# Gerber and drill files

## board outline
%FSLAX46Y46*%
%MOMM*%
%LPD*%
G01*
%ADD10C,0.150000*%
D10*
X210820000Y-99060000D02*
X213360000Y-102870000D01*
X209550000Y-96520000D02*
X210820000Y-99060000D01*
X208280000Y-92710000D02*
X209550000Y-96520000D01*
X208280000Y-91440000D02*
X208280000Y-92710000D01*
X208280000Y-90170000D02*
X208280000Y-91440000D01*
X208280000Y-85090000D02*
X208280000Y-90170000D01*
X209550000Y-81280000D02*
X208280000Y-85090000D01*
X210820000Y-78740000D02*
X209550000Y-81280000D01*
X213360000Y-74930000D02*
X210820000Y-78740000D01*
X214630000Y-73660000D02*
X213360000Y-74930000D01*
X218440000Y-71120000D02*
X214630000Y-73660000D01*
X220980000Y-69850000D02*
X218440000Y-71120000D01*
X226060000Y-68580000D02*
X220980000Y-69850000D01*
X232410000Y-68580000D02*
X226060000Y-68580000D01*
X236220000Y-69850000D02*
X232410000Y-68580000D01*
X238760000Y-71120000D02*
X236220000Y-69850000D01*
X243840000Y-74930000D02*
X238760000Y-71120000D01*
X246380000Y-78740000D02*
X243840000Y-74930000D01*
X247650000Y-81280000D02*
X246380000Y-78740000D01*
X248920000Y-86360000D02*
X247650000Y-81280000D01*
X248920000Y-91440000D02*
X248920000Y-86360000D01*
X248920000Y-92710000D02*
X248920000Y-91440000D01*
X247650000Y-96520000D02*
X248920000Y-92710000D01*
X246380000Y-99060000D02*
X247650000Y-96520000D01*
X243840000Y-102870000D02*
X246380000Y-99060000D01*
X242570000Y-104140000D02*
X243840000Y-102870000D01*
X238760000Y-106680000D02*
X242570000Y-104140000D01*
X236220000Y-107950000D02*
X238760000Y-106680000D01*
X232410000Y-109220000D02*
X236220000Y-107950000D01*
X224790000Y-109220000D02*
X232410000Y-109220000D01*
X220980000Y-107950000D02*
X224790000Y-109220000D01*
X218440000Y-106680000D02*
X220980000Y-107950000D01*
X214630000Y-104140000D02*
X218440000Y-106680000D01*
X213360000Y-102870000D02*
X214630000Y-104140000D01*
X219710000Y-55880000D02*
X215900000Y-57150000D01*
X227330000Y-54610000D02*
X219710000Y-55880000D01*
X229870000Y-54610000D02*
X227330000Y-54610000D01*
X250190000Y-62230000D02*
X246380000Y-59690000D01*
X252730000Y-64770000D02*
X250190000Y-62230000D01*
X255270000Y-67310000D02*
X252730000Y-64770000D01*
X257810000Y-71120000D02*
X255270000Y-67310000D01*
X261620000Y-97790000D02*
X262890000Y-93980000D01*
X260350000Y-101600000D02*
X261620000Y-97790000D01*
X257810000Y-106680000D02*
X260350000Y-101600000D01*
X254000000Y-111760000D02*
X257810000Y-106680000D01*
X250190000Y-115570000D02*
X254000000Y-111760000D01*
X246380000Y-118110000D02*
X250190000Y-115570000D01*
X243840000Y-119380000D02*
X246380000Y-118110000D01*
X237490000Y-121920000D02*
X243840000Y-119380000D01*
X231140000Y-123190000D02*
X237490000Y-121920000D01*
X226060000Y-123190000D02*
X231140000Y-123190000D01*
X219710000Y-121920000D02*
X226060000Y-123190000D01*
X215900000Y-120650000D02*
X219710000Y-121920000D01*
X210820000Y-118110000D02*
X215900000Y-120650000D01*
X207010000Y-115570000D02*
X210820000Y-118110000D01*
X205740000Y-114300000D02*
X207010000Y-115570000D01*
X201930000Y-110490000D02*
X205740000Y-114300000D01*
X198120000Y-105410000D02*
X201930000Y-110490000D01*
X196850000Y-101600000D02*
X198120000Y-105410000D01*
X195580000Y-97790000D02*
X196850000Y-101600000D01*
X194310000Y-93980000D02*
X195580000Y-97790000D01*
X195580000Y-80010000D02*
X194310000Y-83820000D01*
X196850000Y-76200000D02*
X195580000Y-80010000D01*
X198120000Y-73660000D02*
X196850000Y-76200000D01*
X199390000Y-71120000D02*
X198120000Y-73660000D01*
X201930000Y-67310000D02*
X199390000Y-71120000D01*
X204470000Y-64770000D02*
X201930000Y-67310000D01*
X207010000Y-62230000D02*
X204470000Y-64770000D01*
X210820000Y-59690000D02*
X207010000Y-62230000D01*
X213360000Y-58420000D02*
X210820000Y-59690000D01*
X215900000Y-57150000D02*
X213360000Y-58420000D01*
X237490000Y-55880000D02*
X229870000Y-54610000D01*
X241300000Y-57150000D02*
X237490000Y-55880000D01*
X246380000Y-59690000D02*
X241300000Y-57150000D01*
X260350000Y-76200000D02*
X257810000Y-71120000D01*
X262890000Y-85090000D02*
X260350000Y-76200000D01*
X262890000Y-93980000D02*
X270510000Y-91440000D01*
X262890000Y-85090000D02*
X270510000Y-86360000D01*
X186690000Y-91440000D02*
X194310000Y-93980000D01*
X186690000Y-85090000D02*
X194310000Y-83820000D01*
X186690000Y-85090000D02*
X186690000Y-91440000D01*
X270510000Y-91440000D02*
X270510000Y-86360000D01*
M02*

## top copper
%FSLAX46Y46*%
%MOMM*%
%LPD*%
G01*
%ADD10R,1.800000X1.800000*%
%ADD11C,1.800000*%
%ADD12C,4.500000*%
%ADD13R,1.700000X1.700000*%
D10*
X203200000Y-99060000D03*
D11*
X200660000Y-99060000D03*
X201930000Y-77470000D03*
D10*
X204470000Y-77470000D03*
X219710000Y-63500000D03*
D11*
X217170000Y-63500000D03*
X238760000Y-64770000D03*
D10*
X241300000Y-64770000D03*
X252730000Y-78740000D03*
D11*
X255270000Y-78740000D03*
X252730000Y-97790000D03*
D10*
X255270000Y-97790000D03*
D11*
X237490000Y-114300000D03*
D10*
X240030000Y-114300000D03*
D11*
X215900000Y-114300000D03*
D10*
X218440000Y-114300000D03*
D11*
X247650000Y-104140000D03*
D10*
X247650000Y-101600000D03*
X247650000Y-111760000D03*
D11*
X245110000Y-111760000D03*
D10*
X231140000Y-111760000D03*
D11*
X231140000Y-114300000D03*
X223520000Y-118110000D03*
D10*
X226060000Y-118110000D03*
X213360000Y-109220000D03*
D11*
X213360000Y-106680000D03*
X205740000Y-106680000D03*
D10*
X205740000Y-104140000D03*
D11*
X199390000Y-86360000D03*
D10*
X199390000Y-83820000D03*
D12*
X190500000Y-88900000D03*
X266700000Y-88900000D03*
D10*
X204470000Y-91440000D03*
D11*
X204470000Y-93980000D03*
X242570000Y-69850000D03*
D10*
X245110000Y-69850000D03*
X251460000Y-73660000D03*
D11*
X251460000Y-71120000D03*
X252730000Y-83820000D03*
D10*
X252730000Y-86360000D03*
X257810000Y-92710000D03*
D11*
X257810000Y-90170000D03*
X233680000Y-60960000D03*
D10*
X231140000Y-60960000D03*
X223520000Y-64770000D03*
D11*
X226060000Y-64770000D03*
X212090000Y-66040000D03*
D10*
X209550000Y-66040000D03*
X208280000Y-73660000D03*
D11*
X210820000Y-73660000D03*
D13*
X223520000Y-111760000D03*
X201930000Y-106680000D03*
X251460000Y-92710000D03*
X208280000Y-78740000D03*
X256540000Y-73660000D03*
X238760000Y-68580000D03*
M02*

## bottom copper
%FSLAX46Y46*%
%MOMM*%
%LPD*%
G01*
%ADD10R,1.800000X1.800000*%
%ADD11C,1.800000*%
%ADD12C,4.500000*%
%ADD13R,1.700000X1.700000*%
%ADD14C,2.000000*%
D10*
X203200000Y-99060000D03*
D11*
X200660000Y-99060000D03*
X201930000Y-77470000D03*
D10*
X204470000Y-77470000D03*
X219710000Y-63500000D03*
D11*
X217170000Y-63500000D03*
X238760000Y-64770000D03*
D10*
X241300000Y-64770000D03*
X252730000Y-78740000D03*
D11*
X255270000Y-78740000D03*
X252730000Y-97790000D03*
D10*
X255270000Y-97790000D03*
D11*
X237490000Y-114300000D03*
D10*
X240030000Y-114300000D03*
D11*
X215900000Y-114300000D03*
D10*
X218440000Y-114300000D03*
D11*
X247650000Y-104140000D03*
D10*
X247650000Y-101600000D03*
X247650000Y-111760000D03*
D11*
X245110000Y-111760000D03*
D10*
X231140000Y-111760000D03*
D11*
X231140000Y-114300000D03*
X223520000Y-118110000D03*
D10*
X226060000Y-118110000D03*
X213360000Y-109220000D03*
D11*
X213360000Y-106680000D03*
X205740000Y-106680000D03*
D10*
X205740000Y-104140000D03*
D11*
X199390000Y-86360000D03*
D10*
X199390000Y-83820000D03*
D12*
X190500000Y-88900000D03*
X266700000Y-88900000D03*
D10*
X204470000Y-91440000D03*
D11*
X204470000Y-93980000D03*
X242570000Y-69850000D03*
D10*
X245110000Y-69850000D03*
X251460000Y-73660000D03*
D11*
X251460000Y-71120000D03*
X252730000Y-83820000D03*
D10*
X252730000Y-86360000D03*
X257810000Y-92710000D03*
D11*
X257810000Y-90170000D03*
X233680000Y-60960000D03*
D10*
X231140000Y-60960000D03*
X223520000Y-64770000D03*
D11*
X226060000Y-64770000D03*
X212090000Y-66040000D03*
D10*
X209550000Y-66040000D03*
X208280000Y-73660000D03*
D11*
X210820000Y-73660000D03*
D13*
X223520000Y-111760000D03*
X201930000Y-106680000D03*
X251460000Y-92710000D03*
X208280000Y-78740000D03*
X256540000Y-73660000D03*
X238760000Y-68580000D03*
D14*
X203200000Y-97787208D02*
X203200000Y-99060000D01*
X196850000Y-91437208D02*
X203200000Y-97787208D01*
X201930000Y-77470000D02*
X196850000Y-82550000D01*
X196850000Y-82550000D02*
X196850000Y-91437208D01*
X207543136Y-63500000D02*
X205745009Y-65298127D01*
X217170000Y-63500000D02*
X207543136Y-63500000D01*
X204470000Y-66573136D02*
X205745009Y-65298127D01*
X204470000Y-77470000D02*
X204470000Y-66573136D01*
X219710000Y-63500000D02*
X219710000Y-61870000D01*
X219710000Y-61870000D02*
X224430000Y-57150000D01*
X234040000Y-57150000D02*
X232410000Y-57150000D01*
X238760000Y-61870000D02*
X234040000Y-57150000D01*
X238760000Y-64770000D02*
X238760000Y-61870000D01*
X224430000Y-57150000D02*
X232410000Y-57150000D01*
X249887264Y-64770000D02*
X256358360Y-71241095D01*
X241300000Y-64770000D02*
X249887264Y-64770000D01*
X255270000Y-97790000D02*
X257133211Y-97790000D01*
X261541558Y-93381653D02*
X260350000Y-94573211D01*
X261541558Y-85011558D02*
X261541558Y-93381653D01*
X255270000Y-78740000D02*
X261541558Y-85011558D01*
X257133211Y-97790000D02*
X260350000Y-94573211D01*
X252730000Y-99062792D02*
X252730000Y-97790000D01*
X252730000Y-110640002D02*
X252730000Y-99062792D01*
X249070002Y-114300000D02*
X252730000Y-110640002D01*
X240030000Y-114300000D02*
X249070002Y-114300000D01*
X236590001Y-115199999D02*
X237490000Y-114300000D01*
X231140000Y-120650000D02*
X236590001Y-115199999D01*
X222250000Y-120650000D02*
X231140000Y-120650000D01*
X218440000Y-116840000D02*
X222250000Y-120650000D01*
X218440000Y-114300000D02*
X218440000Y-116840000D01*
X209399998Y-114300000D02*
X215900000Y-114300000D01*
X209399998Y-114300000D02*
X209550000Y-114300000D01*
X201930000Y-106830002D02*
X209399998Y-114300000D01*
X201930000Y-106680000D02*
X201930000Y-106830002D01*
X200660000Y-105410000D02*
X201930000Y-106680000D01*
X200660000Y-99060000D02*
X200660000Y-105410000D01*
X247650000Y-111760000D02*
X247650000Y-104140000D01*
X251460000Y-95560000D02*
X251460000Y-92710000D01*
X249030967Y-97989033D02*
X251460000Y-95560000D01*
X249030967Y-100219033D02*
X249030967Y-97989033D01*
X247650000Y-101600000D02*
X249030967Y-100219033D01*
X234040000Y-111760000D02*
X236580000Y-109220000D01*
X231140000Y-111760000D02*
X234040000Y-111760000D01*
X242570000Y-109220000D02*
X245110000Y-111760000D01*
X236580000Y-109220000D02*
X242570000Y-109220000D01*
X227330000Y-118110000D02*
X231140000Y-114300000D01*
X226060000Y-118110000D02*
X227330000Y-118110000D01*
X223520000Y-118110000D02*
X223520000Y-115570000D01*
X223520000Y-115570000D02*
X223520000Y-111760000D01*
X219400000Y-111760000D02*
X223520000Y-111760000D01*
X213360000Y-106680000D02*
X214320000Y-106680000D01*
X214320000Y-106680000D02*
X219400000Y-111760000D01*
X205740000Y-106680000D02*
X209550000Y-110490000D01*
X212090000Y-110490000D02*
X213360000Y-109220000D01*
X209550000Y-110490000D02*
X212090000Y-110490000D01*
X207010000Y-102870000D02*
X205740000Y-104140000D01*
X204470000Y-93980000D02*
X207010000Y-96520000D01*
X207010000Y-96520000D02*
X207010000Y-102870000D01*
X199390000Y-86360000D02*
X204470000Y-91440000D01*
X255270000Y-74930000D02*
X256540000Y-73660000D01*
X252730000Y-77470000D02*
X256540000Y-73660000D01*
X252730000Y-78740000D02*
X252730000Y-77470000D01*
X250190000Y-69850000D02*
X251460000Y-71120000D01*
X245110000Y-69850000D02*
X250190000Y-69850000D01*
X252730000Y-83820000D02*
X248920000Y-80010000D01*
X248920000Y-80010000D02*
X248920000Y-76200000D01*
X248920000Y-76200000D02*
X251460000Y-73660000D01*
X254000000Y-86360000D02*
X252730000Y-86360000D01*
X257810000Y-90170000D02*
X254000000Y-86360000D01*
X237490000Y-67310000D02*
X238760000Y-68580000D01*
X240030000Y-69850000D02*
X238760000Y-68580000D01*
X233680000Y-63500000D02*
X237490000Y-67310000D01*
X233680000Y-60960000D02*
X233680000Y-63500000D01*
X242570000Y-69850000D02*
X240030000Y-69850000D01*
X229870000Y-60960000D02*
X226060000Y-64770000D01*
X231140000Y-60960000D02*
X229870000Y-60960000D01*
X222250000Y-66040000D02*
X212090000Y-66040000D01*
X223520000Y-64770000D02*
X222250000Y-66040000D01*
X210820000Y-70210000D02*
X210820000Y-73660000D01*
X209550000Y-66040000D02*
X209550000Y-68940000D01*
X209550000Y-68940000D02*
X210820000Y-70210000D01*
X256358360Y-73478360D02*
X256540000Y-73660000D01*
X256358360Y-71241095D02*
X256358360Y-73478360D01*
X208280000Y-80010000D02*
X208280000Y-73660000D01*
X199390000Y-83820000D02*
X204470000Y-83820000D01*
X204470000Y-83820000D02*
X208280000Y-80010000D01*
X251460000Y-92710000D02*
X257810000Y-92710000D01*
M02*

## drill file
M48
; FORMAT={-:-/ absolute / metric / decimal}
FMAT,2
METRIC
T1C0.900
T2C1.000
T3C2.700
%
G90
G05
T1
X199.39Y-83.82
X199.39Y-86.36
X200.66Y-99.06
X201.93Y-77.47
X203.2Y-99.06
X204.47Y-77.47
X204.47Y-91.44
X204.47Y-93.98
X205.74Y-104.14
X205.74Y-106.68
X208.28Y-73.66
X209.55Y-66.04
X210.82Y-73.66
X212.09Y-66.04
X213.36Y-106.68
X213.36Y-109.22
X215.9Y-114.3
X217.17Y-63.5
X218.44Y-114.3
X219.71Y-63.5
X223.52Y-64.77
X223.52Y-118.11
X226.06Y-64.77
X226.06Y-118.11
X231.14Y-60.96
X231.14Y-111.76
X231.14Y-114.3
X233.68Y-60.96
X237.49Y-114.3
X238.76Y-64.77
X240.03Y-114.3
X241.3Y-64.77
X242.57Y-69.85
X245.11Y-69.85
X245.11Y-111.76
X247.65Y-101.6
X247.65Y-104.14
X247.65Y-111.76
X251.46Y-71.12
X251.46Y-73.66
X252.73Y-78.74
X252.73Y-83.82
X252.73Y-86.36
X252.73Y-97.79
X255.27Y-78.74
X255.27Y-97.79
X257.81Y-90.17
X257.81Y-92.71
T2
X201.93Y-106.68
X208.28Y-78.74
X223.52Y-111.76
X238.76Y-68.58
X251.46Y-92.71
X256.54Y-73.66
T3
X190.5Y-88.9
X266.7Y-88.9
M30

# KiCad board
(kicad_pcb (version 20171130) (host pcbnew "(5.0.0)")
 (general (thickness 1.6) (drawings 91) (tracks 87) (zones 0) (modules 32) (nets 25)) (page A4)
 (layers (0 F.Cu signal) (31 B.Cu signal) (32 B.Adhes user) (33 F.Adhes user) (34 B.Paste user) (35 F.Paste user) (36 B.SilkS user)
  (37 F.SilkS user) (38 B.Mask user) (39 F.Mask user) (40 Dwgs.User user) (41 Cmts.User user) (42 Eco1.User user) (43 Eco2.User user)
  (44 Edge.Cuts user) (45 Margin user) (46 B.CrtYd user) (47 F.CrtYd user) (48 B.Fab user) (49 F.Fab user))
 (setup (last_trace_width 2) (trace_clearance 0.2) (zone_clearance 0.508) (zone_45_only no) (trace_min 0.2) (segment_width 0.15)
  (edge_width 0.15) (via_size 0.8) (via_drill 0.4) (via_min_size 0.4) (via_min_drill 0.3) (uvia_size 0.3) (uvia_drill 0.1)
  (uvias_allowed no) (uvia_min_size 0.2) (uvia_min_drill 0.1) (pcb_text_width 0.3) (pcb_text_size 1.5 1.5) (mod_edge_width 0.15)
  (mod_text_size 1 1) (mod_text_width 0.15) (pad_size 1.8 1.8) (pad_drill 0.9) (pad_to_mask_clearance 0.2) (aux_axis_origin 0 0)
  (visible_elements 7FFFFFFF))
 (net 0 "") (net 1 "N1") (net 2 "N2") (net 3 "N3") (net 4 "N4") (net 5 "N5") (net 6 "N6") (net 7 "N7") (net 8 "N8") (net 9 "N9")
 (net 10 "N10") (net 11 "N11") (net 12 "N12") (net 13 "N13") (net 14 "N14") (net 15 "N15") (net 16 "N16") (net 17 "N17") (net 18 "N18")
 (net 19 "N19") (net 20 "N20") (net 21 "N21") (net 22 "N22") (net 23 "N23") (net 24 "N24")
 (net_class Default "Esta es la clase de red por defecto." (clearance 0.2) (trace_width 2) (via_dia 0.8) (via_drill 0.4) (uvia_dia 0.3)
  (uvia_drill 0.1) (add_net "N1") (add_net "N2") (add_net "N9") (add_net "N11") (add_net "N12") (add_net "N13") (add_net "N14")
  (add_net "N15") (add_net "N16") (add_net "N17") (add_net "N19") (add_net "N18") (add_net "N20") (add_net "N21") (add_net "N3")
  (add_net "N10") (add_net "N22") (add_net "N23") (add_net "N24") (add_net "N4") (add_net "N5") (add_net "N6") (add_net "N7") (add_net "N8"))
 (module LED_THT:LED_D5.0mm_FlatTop (layer F.Cu) (at 203.2 99.06 180)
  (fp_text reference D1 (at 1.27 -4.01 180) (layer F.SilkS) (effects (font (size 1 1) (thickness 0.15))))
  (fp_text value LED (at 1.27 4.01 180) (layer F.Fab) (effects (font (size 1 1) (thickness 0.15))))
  (pad 1 thru_hole rect (at 0 0 180) (size 1.8 1.8) (drill 0.9) (layers *.Cu *.Mask) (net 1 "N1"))
  (pad 2 thru_hole circle (at 2.54 0 180) (size 1.8 1.8) (drill 0.9) (layers *.Cu *.Mask) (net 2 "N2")))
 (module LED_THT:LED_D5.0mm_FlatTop (layer F.Cu) (at 204.47 77.47 180)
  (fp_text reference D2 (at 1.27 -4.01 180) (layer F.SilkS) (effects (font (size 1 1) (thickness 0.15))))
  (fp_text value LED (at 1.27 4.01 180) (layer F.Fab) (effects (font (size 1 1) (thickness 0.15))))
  (pad 2 thru_hole circle (at 2.54 0 180) (size 1.8 1.8) (drill 0.9) (layers *.Cu *.Mask) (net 1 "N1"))
  (pad 1 thru_hole rect (at 0 0 180) (size 1.8 1.8) (drill 0.9) (layers *.Cu *.Mask) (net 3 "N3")))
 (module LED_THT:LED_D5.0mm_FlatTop (layer F.Cu) (at 219.71 63.5 180)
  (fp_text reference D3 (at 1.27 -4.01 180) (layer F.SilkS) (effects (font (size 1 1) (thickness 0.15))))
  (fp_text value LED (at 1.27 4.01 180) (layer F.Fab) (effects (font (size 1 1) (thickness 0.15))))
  (pad 1 thru_hole rect (at 0 0 180) (size 1.8 1.8) (drill 0.9) (layers *.Cu *.Mask) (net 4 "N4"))
  (pad 2 thru_hole circle (at 2.54 0 180) (size 1.8 1.8) (drill 0.9) (layers *.Cu *.Mask) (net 3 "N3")))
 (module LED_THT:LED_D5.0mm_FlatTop (layer F.Cu) (at 241.3 64.77 180)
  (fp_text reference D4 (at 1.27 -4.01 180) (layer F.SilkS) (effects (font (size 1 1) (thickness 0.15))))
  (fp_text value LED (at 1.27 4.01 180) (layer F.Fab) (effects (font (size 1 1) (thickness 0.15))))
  (pad 2 thru_hole circle (at 2.54 0 180) (size 1.8 1.8) (drill 0.9) (layers *.Cu *.Mask) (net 4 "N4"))
  (pad 1 thru_hole rect (at 0 0 180) (size 1.8 1.8) (drill 0.9) (layers *.Cu *.Mask) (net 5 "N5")))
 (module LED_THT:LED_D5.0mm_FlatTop (layer F.Cu) (at 252.73 78.74)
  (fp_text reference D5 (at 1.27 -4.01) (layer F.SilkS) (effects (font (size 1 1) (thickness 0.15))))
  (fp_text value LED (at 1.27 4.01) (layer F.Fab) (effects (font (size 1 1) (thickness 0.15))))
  (pad 1 thru_hole rect (at 0 0) (size 1.8 1.8) (drill 0.9) (layers *.Cu *.Mask) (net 5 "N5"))
  (pad 2 thru_hole circle (at 2.54 0) (size 1.8 1.8) (drill 0.9) (layers *.Cu *.Mask) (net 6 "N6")))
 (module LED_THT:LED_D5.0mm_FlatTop (layer F.Cu) (at 255.27 97.79 180)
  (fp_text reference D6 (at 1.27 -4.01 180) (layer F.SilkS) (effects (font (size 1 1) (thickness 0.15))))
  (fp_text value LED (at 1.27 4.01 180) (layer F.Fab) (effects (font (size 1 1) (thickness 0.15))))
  (pad 2 thru_hole circle (at 2.54 0 180) (size 1.8 1.8) (drill 0.9) (layers *.Cu *.Mask) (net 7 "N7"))
  (pad 1 thru_hole rect (at 0 0 180) (size 1.8 1.8) (drill 0.9) (layers *.Cu *.Mask) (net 6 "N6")))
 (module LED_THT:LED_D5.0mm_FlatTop (layer F.Cu) (at 240.03 114.3 180)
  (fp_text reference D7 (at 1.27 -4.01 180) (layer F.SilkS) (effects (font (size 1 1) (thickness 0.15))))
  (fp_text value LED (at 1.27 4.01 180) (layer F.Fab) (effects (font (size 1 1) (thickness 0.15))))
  (pad 2 thru_hole circle (at 2.54 0 180) (size 1.8 1.8) (drill 0.9) (layers *.Cu *.Mask) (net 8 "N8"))
  (pad 1 thru_hole rect (at 0 0 180) (size 1.8 1.8) (drill 0.9) (layers *.Cu *.Mask) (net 7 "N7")))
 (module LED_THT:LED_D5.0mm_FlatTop (layer F.Cu) (at 218.44 114.3 180)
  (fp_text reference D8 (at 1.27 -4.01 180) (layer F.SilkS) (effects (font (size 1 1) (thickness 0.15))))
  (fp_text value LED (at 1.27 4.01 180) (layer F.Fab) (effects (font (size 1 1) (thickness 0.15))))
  (pad 2 thru_hole circle (at 2.54 0 180) (size 1.8 1.8) (drill 0.9) (layers *.Cu *.Mask) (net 2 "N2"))
  (pad 1 thru_hole rect (at 0 0 180) (size 1.8 1.8) (drill 0.9) (layers *.Cu *.Mask) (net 8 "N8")))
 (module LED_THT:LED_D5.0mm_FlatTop (layer F.Cu) (at 247.65 101.6 270)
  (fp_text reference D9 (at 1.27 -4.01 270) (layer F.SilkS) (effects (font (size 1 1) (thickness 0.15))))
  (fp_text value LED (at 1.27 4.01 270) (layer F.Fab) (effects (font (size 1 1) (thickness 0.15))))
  (pad 2 thru_hole circle (at 2.54 0 270) (size 1.8 1.8) (drill 0.9) (layers *.Cu *.Mask) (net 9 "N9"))
  (pad 1 thru_hole rect (at 0 0 270) (size 1.8 1.8) (drill 0.9) (layers *.Cu *.Mask) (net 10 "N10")))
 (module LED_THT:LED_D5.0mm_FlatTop (layer F.Cu) (at 247.65 111.76 180)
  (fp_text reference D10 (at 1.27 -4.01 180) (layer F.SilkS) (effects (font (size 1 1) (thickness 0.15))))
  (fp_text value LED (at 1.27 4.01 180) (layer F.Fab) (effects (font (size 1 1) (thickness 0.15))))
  (pad 1 thru_hole rect (at 0 0 180) (size 1.8 1.8) (drill 0.9) (layers *.Cu *.Mask) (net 9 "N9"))
  (pad 2 thru_hole circle (at 2.54 0 180) (size 1.8 1.8) (drill 0.9) (layers *.Cu *.Mask) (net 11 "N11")))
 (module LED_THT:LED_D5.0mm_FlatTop (layer F.Cu) (at 231.14 111.76 270)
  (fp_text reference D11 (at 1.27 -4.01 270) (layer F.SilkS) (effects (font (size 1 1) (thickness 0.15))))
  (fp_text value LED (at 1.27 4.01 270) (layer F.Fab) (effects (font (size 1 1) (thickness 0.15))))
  (pad 1 thru_hole rect (at 0 0 270) (size 1.8 1.8) (drill 0.9) (layers *.Cu *.Mask) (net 11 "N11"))
  (pad 2 thru_hole circle (at 2.54 0 270) (size 1.8 1.8) (drill 0.9) (layers *.Cu *.Mask) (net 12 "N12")))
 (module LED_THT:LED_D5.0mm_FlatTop (layer F.Cu) (at 226.06 118.11 180)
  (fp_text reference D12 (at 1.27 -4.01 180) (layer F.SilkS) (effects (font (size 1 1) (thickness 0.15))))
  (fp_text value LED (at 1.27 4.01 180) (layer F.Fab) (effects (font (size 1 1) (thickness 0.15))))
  (pad 2 thru_hole circle (at 2.54 0 180) (size 1.8 1.8) (drill 0.9) (layers *.Cu *.Mask) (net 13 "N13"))
  (pad 1 thru_hole rect (at 0 0 180) (size 1.8 1.8) (drill 0.9) (layers *.Cu *.Mask) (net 12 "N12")))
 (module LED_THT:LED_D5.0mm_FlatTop (layer F.Cu) (at 213.36 109.22 90)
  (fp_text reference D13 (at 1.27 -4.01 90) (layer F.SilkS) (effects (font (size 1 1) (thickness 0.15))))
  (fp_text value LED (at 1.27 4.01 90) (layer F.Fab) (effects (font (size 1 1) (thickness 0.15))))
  (pad 1 thru_hole rect (at 0 0 90) (size 1.8 1.8) (drill 0.9) (layers *.Cu *.Mask) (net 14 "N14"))
  (pad 2 thru_hole circle (at 2.54 0 90) (size 1.8 1.8) (drill 0.9) (layers *.Cu *.Mask) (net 13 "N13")))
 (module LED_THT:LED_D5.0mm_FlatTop (layer F.Cu) (at 205.74 104.14 270)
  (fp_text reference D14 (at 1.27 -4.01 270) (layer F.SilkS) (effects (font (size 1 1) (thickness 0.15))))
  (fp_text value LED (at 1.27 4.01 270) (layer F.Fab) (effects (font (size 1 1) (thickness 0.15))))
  (pad 2 thru_hole circle (at 2.54 0 270) (size 1.8 1.8) (drill 0.9) (layers *.Cu *.Mask) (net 14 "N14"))
  (pad 1 thru_hole rect (at 0 0 270) (size 1.8 1.8) (drill 0.9) (layers *.Cu *.Mask) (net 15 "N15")))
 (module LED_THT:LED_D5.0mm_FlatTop (layer F.Cu) (at 199.39 83.82 270)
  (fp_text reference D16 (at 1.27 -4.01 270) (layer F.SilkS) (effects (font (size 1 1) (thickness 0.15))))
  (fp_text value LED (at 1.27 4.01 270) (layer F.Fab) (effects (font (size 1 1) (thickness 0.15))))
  (pad 2 thru_hole circle (at 2.54 0 270) (size 1.8 1.8) (drill 0.9) (layers *.Cu *.Mask) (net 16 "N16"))
  (pad 1 thru_hole rect (at 0 0 270) (size 1.8 1.8) (drill 0.9) (layers *.Cu *.Mask) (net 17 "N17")))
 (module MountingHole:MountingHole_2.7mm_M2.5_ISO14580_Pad (layer F.Cu) (at 190.5 88.9)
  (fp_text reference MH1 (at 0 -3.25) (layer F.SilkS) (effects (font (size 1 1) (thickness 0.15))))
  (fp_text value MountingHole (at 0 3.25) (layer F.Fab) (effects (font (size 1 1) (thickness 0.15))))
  (pad 1 thru_hole circle (at 0 0) (size 4.5 4.5) (drill 2.7) (layers *.Cu *.Mask)))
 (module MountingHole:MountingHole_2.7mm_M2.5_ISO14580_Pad (layer F.Cu) (at 266.7 88.9)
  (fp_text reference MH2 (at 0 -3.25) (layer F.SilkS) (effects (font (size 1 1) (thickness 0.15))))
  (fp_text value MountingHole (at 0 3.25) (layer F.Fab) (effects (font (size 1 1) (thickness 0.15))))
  (pad 1 thru_hole circle (at 0 0) (size 4.5 4.5) (drill 2.7) (layers *.Cu *.Mask)))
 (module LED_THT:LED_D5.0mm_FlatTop (layer F.Cu) (at 204.47 91.44 270)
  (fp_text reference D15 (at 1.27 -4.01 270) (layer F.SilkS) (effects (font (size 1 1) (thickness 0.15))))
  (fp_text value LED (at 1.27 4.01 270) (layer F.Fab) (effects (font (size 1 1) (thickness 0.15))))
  (pad 1 thru_hole rect (at 0 0 270) (size 1.8 1.8) (drill 0.9) (layers *.Cu *.Mask) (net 16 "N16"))
  (pad 2 thru_hole circle (at 2.54 0 270) (size 1.8 1.8) (drill 0.9) (layers *.Cu *.Mask) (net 15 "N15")))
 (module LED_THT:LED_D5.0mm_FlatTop (layer F.Cu) (at 245.11 69.85 180)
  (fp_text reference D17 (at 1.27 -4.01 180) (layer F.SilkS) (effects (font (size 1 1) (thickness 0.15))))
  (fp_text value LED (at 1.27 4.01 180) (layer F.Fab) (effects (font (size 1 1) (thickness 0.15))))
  (pad 2 thru_hole circle (at 2.54 0 180) (size 1.8 1.8) (drill 0.9) (layers *.Cu *.Mask) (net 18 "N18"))
  (pad 1 thru_hole rect (at 0 0 180) (size 1.8 1.8) (drill 0.9) (layers *.Cu *.Mask) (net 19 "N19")))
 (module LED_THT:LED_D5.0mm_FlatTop (layer F.Cu) (at 251.46 73.66 90)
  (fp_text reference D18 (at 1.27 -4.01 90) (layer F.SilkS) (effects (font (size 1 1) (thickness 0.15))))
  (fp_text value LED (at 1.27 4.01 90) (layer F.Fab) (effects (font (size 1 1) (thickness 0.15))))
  (pad 1 thru_hole rect (at 0 0 90) (size 1.8 1.8) (drill 0.9) (layers *.Cu *.Mask) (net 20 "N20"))
  (pad 2 thru_hole circle (at 2.54 0 90) (size 1.8 1.8) (drill 0.9) (layers *.Cu *.Mask) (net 19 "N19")))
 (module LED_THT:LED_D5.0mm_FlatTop (layer F.Cu) (at 252.73 86.36 90)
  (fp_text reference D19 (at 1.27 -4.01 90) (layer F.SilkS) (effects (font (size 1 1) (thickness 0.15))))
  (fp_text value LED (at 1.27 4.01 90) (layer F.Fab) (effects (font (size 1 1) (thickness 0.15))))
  (pad 2 thru_hole circle (at 2.54 0 90) (size 1.8 1.8) (drill 0.9) (layers *.Cu *.Mask) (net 20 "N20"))
  (pad 1 thru_hole rect (at 0 0 90) (size 1.8 1.8) (drill 0.9) (layers *.Cu *.Mask) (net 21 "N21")))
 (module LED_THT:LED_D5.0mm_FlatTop (layer F.Cu) (at 257.81 92.71 90)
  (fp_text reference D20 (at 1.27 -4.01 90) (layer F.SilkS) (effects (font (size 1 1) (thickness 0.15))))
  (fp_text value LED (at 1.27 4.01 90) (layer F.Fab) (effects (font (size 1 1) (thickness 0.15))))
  (pad 1 thru_hole rect (at 0 0 90) (size 1.8 1.8) (drill 0.9) (layers *.Cu *.Mask) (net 10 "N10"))
  (pad 2 thru_hole circle (at 2.54 0 90) (size 1.8 1.8) (drill 0.9) (layers *.Cu *.Mask) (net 21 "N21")))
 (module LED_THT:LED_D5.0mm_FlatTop (layer F.Cu) (at 231.14 60.96)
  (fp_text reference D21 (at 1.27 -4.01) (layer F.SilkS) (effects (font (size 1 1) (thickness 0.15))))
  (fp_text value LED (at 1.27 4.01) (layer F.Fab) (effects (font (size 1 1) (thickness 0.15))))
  (pad 2 thru_hole circle (at 2.54 0) (size 1.8 1.8) (drill 0.9) (layers *.Cu *.Mask) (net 18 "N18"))
  (pad 1 thru_hole rect (at 0 0) (size 1.8 1.8) (drill 0.9) (layers *.Cu *.Mask) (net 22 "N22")))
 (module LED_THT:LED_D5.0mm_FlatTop (layer F.Cu) (at 223.52 64.77)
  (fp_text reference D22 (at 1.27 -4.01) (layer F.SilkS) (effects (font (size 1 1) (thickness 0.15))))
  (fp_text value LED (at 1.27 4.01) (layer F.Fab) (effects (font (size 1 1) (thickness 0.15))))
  (pad 1 thru_hole rect (at 0 0) (size 1.8 1.8) (drill 0.9) (layers *.Cu *.Mask) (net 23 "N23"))
  (pad 2 thru_hole circle (at 2.54 0) (size 1.8 1.8) (drill 0.9) (layers *.Cu *.Mask) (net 22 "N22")))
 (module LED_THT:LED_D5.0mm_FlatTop (layer F.Cu) (at 209.55 66.04)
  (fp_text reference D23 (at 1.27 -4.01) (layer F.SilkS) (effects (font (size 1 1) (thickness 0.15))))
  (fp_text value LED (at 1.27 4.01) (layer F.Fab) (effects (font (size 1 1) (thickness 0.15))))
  (pad 2 thru_hole circle (at 2.54 0) (size 1.8 1.8) (drill 0.9) (layers *.Cu *.Mask) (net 23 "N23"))
  (pad 1 thru_hole rect (at 0 0) (size 1.8 1.8) (drill 0.9) (layers *.Cu *.Mask) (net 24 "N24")))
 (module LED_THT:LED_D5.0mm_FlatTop (layer F.Cu) (at 208.28 73.66)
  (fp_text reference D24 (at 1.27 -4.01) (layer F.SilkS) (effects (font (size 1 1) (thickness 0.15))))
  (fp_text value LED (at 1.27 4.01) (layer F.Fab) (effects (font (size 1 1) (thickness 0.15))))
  (pad 1 thru_hole rect (at 0 0) (size 1.8 1.8) (drill 0.9) (layers *.Cu *.Mask) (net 17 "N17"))
  (pad 2 thru_hole circle (at 2.54 0) (size 1.8 1.8) (drill 0.9) (layers *.Cu *.Mask) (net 24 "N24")))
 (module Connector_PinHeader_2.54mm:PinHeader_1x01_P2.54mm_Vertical (layer F.Cu) (at 223.52 111.76 180)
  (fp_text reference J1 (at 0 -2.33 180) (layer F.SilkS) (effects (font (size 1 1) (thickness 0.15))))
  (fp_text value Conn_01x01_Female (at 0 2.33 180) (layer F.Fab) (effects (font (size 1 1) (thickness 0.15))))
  (pad 1 thru_hole rect (at 0 0 180) (size 1.7 1.7) (drill 1) (layers *.Cu *.Mask) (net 13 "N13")))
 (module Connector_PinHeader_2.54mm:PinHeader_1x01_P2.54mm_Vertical (layer F.Cu) (at 201.93 106.68)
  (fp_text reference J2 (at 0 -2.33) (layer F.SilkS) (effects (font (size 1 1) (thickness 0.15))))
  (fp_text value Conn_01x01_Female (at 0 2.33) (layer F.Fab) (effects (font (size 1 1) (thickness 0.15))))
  (pad 1 thru_hole rect (at 0 0) (size 1.7 1.7) (drill 1) (layers *.Cu *.Mask) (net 2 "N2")))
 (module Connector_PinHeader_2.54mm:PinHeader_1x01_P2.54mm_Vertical (layer F.Cu) (at 251.46 92.71 90)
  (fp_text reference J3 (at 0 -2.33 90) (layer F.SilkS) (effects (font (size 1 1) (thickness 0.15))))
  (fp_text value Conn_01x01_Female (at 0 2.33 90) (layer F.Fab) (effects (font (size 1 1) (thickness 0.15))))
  (pad 1 thru_hole rect (at 0 0 90) (size 1.7 1.7) (drill 1) (layers *.Cu *.Mask) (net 10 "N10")))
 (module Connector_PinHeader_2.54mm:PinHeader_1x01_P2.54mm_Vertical (layer F.Cu) (at 208.28 78.74)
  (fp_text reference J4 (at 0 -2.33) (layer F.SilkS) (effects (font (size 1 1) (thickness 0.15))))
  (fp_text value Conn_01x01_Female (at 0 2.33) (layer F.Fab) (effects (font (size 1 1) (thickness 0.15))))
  (pad 1 thru_hole rect (at 0 0) (size 1.7 1.7) (drill 1) (layers *.Cu *.Mask) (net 17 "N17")))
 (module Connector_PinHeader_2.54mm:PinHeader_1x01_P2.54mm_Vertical (layer F.Cu) (at 256.54 73.66 180)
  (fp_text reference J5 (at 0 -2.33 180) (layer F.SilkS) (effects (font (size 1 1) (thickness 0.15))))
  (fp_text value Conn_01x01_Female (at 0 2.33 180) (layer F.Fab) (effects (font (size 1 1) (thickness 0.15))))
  (pad 1 thru_hole rect (at 0 0 180) (size 1.7 1.7) (drill 1) (layers *.Cu *.Mask) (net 5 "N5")))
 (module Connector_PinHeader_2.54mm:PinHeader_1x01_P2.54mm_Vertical (layer F.Cu) (at 238.76 68.58 270)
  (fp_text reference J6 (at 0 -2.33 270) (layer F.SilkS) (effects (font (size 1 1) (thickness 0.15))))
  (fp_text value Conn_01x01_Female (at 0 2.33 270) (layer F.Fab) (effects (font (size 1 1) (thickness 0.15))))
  (pad 1 thru_hole rect (at 0 0 270) (size 1.7 1.7) (drill 1) (layers *.Cu *.Mask) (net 18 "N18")))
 (gr_line (start 210.82 99.06) (end 213.36 102.87) (layer Edge.Cuts) (width 0.15))
 (gr_line (start 209.55 96.52) (end 210.82 99.06) (layer Edge.Cuts) (width 0.15))
 (gr_line (start 208.28 92.71) (end 209.55 96.52) (layer Edge.Cuts) (width 0.15))
 (gr_line (start 208.28 91.44) (end 208.28 92.71) (layer Edge.Cuts) (width 0.15))
 (gr_line (start 208.28 90.17) (end 208.28 91.44) (layer Edge.Cuts) (width 0.15))
 (gr_line (start 208.28 85.09) (end 208.28 90.17) (layer Edge.Cuts) (width 0.15))
 (gr_line (start 209.55 81.28) (end 208.28 85.09) (layer Edge.Cuts) (width 0.15))
 (gr_line (start 210.82 78.74) (end 209.55 81.28) (layer Edge.Cuts) (width 0.15))
 (gr_line (start 213.36 74.93) (end 210.82 78.74) (layer Edge.Cuts) (width 0.15))
 (gr_line (start 214.63 73.66) (end 213.36 74.93) (layer Edge.Cuts) (width 0.15))
 (gr_line (start 218.44 71.12) (end 214.63 73.66) (layer Edge.Cuts) (width 0.15))
 (gr_line (start 220.98 69.85) (end 218.44 71.12) (layer Edge.Cuts) (width 0.15))
 (gr_line (start 226.06 68.58) (end 220.98 69.85) (layer Edge.Cuts) (width 0.15))
 (gr_line (start 232.41 68.58) (end 226.06 68.58) (layer Edge.Cuts) (width 0.15))
 (gr_line (start 236.22 69.85) (end 232.41 68.58) (layer Edge.Cuts) (width 0.15))
 (gr_line (start 238.76 71.12) (end 236.22 69.85) (layer Edge.Cuts) (width 0.15))
 (gr_line (start 243.84 74.93) (end 238.76 71.12) (layer Edge.Cuts) (width 0.15))
 (gr_line (start 246.38 78.74) (end 243.84 74.93) (layer Edge.Cuts) (width 0.15))
 (gr_line (start 247.65 81.28) (end 246.38 78.74) (layer Edge.Cuts) (width 0.15))
 (gr_line (start 248.92 86.36) (end 247.65 81.28) (layer Edge.Cuts) (width 0.15))
 (gr_line (start 248.92 91.44) (end 248.92 86.36) (layer Edge.Cuts) (width 0.15))
 (gr_line (start 248.92 92.71) (end 248.92 91.44) (layer Edge.Cuts) (width 0.15))
 (gr_line (start 247.65 96.52) (end 248.92 92.71) (layer Edge.Cuts) (width 0.15))
 (gr_line (start 246.38 99.06) (end 247.65 96.52) (layer Edge.Cuts) (width 0.15))
 (gr_line (start 243.84 102.87) (end 246.38 99.06) (layer Edge.Cuts) (width 0.15))
 (gr_line (start 242.57 104.14) (end 243.84 102.87) (layer Edge.Cuts) (width 0.15))
 (gr_line (start 238.76 106.68) (end 242.57 104.14) (layer Edge.Cuts) (width 0.15))
 (gr_line (start 236.22 107.95) (end 238.76 106.68) (layer Edge.Cuts) (width 0.15))
 (gr_line (start 232.41 109.22) (end 236.22 107.95) (layer Edge.Cuts) (width 0.15))
 (gr_line (start 224.79 109.22) (end 232.41 109.22) (layer Edge.Cuts) (width 0.15))
 (gr_line (start 220.98 107.95) (end 224.79 109.22) (layer Edge.Cuts) (width 0.15))
 (gr_line (start 218.44 106.68) (end 220.98 107.95) (layer Edge.Cuts) (width 0.15))
 (gr_line (start 214.63 104.14) (end 218.44 106.68) (layer Edge.Cuts) (width 0.15))
 (gr_line (start 213.36 102.87) (end 214.63 104.14) (layer Edge.Cuts) (width 0.15))
 (gr_line (start 219.71 55.88) (end 215.9 57.15) (layer Edge.Cuts) (width 0.15))
 (gr_line (start 227.33 54.61) (end 219.71 55.88) (layer Edge.Cuts) (width 0.15))
 (gr_line (start 229.87 54.61) (end 227.33 54.61) (layer Edge.Cuts) (width 0.15))
 (gr_line (start 250.19 62.23) (end 246.38 59.69) (layer Edge.Cuts) (width 0.15))
 (gr_line (start 252.73 64.77) (end 250.19 62.23) (layer Edge.Cuts) (width 0.15))
 (gr_line (start 255.27 67.31) (end 252.73 64.77) (layer Edge.Cuts) (width 0.15))
 (gr_line (start 257.81 71.12) (end 255.27 67.31) (layer Edge.Cuts) (width 0.15))
 (gr_line (start 261.62 97.79) (end 262.89 93.98) (layer Edge.Cuts) (width 0.15))
 (gr_line (start 260.35 101.6) (end 261.62 97.79) (layer Edge.Cuts) (width 0.15))
 (gr_line (start 257.81 106.68) (end 260.35 101.6) (layer Edge.Cuts) (width 0.15))
 (gr_line (start 254 111.76) (end 257.81 106.68) (layer Edge.Cuts) (width 0.15))
 (gr_line (start 250.19 115.57) (end 254 111.76) (layer Edge.Cuts) (width 0.15))
 (gr_line (start 246.38 118.11) (end 250.19 115.57) (layer Edge.Cuts) (width 0.15))
 (gr_line (start 243.84 119.38) (end 246.38 118.11) (layer Edge.Cuts) (width 0.15))
 (gr_line (start 237.49 121.92) (end 243.84 119.38) (layer Edge.Cuts) (width 0.15))
 (gr_line (start 231.14 123.19) (end 237.49 121.92) (layer Edge.Cuts) (width 0.15))
 (gr_line (start 226.06 123.19) (end 231.14 123.19) (layer Edge.Cuts) (width 0.15))
 (gr_line (start 219.71 121.92) (end 226.06 123.19) (layer Edge.Cuts) (width 0.15))
 (gr_line (start 215.9 120.65) (end 219.71 121.92) (layer Edge.Cuts) (width 0.15))
 (gr_line (start 210.82 118.11) (end 215.9 120.65) (layer Edge.Cuts) (width 0.15))
 (gr_line (start 207.01 115.57) (end 210.82 118.11) (layer Edge.Cuts) (width 0.15))
 (gr_line (start 205.74 114.3) (end 207.01 115.57) (layer Edge.Cuts) (width 0.15))
 (gr_line (start 201.93 110.49) (end 205.74 114.3) (layer Edge.Cuts) (width 0.15))
 (gr_line (start 198.12 105.41) (end 201.93 110.49) (layer Edge.Cuts) (width 0.15))
 (gr_line (start 196.85 101.6) (end 198.12 105.41) (layer Edge.Cuts) (width 0.15))
 (gr_line (start 195.58 97.79) (end 196.85 101.6) (layer Edge.Cuts) (width 0.15))
 (gr_line (start 194.31 93.98) (end 195.58 97.79) (layer Edge.Cuts) (width 0.15))
 (gr_line (start 195.58 80.01) (end 194.31 83.82) (layer Edge.Cuts) (width 0.15))
 (gr_line (start 196.85 76.2) (end 195.58 80.01) (layer Edge.Cuts) (width 0.15))
 (gr_line (start 198.12 73.66) (end 196.85 76.2) (layer Edge.Cuts) (width 0.15))
 (gr_line (start 199.39 71.12) (end 198.12 73.66) (layer Edge.Cuts) (width 0.15))
 (gr_line (start 201.93 67.31) (end 199.39 71.12) (layer Edge.Cuts) (width 0.15))
 (gr_line (start 204.47 64.77) (end 201.93 67.31) (layer Edge.Cuts) (width 0.15))
 (gr_line (start 207.01 62.23) (end 204.47 64.77) (layer Edge.Cuts) (width 0.15))
 (gr_line (start 210.82 59.69) (end 207.01 62.23) (layer Edge.Cuts) (width 0.15))
 (gr_line (start 213.36 58.42) (end 210.82 59.69) (layer Edge.Cuts) (width 0.15))
 (gr_line (start 215.9 57.15) (end 213.36 58.42) (layer Edge.Cuts) (width 0.15))
 (gr_line (start 237.49 55.88) (end 229.87 54.61) (layer Edge.Cuts) (width 0.15))
 (gr_line (start 241.3 57.15) (end 237.49 55.88) (layer Edge.Cuts) (width 0.15))
 (gr_line (start 246.38 59.69) (end 241.3 57.15) (layer Edge.Cuts) (width 0.15))
 (gr_line (start 260.35 76.2) (end 257.81 71.12) (layer Edge.Cuts) (width 0.15))
 (gr_line (start 262.89 85.09) (end 260.35 76.2) (layer Edge.Cuts) (width 0.15))
 (gr_line (start 262.89 93.98) (end 270.51 91.44) (layer Edge.Cuts) (width 0.15))
 (gr_line (start 262.89 85.09) (end 270.51 86.36) (layer Edge.Cuts) (width 0.15))
 (gr_line (start 186.69 91.44) (end 194.31 93.98) (layer Edge.Cuts) (width 0.15))
 (gr_line (start 186.69 85.09) (end 194.31 83.82) (layer Edge.Cuts) (width 0.15))
 (gr_line (start 186.69 85.09) (end 186.69 91.44) (layer Edge.Cuts) (width 0.15))
 (gr_line (start 270.51 91.44) (end 270.51 86.36) (layer Edge.Cuts) (width 0.15))
 (segment (start 203.2 97.787208) (end 203.2 99.06) (width 2) (layer B.Cu) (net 1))
 (segment (start 196.85 91.437208) (end 203.2 97.787208) (width 2) (layer B.Cu) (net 1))
 (segment (start 201.93 77.47) (end 196.85 82.55) (width 2) (layer B.Cu) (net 1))
 (segment (start 196.85 82.55) (end 196.85 91.437208) (width 2) (layer B.Cu) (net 1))
 (segment (start 207.543136 63.5) (end 205.745009 65.298127) (width 2) (layer B.Cu) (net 3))
 (segment (start 217.17 63.5) (end 207.543136 63.5) (width 2) (layer B.Cu) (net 3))
 (segment (start 204.47 66.573136) (end 205.745009 65.298127) (width 2) (layer B.Cu) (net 3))
 (segment (start 204.47 77.47) (end 204.47 66.573136) (width 2) (layer B.Cu) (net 3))
 (segment (start 219.71 63.5) (end 219.71 61.87) (width 2) (layer B.Cu) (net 4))
 (segment (start 219.71 61.87) (end 224.43 57.15) (width 2) (layer B.Cu) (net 4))
 (segment (start 234.04 57.15) (end 232.41 57.15) (width 2) (layer B.Cu) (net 4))
 (segment (start 238.76 61.87) (end 234.04 57.15) (width 2) (layer B.Cu) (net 4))
 (segment (start 238.76 64.77) (end 238.76 61.87) (width 2) (layer B.Cu) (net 4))
 (segment (start 224.43 57.15) (end 232.41 57.15) (width 2) (layer B.Cu) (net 4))
 (segment (start 249.887264 64.77) (end 256.35836 71.241095) (width 2) (layer B.Cu) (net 5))
 (segment (start 241.3 64.77) (end 249.887264 64.77) (width 2) (layer B.Cu) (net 5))
 (segment (start 255.27 97.79) (end 257.133211 97.79) (width 2) (layer B.Cu) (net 6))
 (segment (start 261.541558 93.381653) (end 260.35 94.573211) (width 2) (layer B.Cu) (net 6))
 (segment (start 261.541558 85.011558) (end 261.541558 93.381653) (width 2) (layer B.Cu) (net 6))
 (segment (start 255.27 78.74) (end 261.541558 85.011558) (width 2) (layer B.Cu) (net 6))
 (segment (start 257.133211 97.79) (end 260.35 94.573211) (width 2) (layer B.Cu) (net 6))
 (segment (start 252.73 99.062792) (end 252.73 97.79) (width 2) (layer B.Cu) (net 7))
 (segment (start 252.73 110.640002) (end 252.73 99.062792) (width 2) (layer B.Cu) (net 7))
 (segment (start 249.070002 114.3) (end 252.73 110.640002) (width 2) (layer B.Cu) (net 7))
 (segment (start 240.03 114.3) (end 249.070002 114.3) (width 2) (layer B.Cu) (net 7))
 (segment (start 236.590001 115.199999) (end 237.49 114.3) (width 2) (layer B.Cu) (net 8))
 (segment (start 231.14 120.65) (end 236.590001 115.199999) (width 2) (layer B.Cu) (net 8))
 (segment (start 222.25 120.65) (end 231.14 120.65) (width 2) (layer B.Cu) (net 8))
 (segment (start 218.44 116.84) (end 222.25 120.65) (width 2) (layer B.Cu) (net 8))
 (segment (start 218.44 114.3) (end 218.44 116.84) (width 2) (layer B.Cu) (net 8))
 (segment (start 209.399998 114.3) (end 215.9 114.3) (width 2) (layer B.Cu) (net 2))
 (segment (start 209.399998 114.3) (end 209.55 114.3) (width 2) (layer B.Cu) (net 2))
 (segment (start 201.93 106.830002) (end 209.399998 114.3) (width 2) (layer B.Cu) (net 2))
 (segment (start 201.93 106.68) (end 201.93 106.830002) (width 2) (layer B.Cu) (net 2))
 (segment (start 200.66 105.41) (end 201.93 106.68) (width 2) (layer B.Cu) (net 2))
 (segment (start 200.66 99.06) (end 200.66 105.41) (width 2) (layer B.Cu) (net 2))
 (segment (start 247.65 111.76) (end 247.65 104.14) (width 2) (layer B.Cu) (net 9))
 (segment (start 251.46 95.56) (end 251.46 92.71) (width 2) (layer B.Cu) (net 10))
 (segment (start 249.030967 97.989033) (end 251.46 95.56) (width 2) (layer B.Cu) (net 10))
 (segment (start 249.030967 100.219033) (end 249.030967 97.989033) (width 2) (layer B.Cu) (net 10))
 (segment (start 247.65 101.6) (end 249.030967 100.219033) (width 2) (layer B.Cu) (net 10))
 (segment (start 234.04 111.76) (end 236.58 109.22) (width 2) (layer B.Cu) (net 11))
 (segment (start 231.14 111.76) (end 234.04 111.76) (width 2) (layer B.Cu) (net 11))
 (segment (start 242.57 109.22) (end 245.11 111.76) (width 2) (layer B.Cu) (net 11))
 (segment (start 236.58 109.22) (end 242.57 109.22) (width 2) (layer B.Cu) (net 11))
 (segment (start 227.33 118.11) (end 231.14 114.3) (width 2) (layer B.Cu) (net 12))
 (segment (start 226.06 118.11) (end 227.33 118.11) (width 2) (layer B.Cu) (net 12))
 (segment (start 223.52 118.11) (end 223.52 115.57) (width 2) (layer B.Cu) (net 13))
 (segment (start 223.52 115.57) (end 223.52 111.76) (width 2) (layer B.Cu) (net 13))
 (segment (start 219.4 111.76) (end 223.52 111.76) (width 2) (layer B.Cu) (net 13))
 (segment (start 213.36 106.68) (end 214.32 106.68) (width 2) (layer B.Cu) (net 13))
 (segment (start 214.32 106.68) (end 219.4 111.76) (width 2) (layer B.Cu) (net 13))
 (segment (start 205.74 106.68) (end 209.55 110.49) (width 2) (layer B.Cu) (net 14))
 (segment (start 212.09 110.49) (end 213.36 109.22) (width 2) (layer B.Cu) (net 14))
 (segment (start 209.55 110.49) (end 212.09 110.49) (width 2) (layer B.Cu) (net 14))
 (segment (start 207.01 102.87) (end 205.74 104.14) (width 2) (layer B.Cu) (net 15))
 (segment (start 204.47 93.98) (end 207.01 96.52) (width 2) (layer B.Cu) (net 15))
 (segment (start 207.01 96.52) (end 207.01 102.87) (width 2) (layer B.Cu) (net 15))
 (segment (start 199.39 86.36) (end 204.47 91.44) (width 2) (layer B.Cu) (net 16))
 (segment (start 255.27 74.93) (end 256.54 73.66) (width 2) (layer B.Cu) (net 5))
 (segment (start 252.73 77.47) (end 256.54 73.66) (width 2) (layer B.Cu) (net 5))
 (segment (start 252.73 78.74) (end 252.73 77.47) (width 2) (layer B.Cu) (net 5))
 (segment (start 250.19 69.85) (end 251.46 71.12) (width 2) (layer B.Cu) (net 19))
 (segment (start 245.11 69.85) (end 250.19 69.85) (width 2) (layer B.Cu) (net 19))
 (segment (start 252.73 83.82) (end 248.92 80.01) (width 2) (layer B.Cu) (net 20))
 (segment (start 248.92 80.01) (end 248.92 76.2) (width 2) (layer B.Cu) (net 20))
 (segment (start 248.92 76.2) (end 251.46 73.66) (width 2) (layer B.Cu) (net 20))
 (segment (start 254 86.36) (end 252.73 86.36) (width 2) (layer B.Cu) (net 21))
 (segment (start 257.81 90.17) (end 254 86.36) (width 2) (layer B.Cu) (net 21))
 (segment (start 237.49 67.31) (end 238.76 68.58) (width 2) (layer B.Cu) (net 18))
 (segment (start 240.03 69.85) (end 238.76 68.58) (width 2) (layer B.Cu) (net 18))
 (segment (start 233.68 63.5) (end 237.49 67.31) (width 2) (layer B.Cu) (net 18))
 (segment (start 233.68 60.96) (end 233.68 63.5) (width 2) (layer B.Cu) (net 18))
 (segment (start 242.57 69.85) (end 240.03 69.85) (width 2) (layer B.Cu) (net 18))
 (segment (start 229.87 60.96) (end 226.06 64.77) (width 2) (layer B.Cu) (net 22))
 (segment (start 231.14 60.96) (end 229.87 60.96) (width 2) (layer B.Cu) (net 22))
 (segment (start 222.25 66.04) (end 212.09 66.04) (width 2) (layer B.Cu) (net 23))
 (segment (start 223.52 64.77) (end 222.25 66.04) (width 2) (layer B.Cu) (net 23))
 (segment (start 210.82 70.21) (end 210.82 73.66) (width 2) (layer B.Cu) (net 24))
 (segment (start 209.55 66.04) (end 209.55 68.94) (width 2) (layer B.Cu) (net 24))
 (segment (start 209.55 68.94) (end 210.82 70.21) (width 2) (layer B.Cu) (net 24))
 (segment (start 256.35836 73.47836) (end 256.54 73.66) (width 2) (layer B.Cu) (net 5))
 (segment (start 256.35836 71.241095) (end 256.35836 73.47836) (width 2) (layer B.Cu) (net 5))
 (segment (start 208.28 80.01) (end 208.28 73.66) (width 2) (layer B.Cu) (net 17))
 (segment (start 199.39 83.82) (end 204.47 83.82) (width 2) (layer B.Cu) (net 17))
 (segment (start 204.47 83.82) (end 208.28 80.01) (width 2) (layer B.Cu) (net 17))
 (segment (start 251.46 92.71) (end 257.81 92.71) (width 2) (layer B.Cu) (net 10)))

